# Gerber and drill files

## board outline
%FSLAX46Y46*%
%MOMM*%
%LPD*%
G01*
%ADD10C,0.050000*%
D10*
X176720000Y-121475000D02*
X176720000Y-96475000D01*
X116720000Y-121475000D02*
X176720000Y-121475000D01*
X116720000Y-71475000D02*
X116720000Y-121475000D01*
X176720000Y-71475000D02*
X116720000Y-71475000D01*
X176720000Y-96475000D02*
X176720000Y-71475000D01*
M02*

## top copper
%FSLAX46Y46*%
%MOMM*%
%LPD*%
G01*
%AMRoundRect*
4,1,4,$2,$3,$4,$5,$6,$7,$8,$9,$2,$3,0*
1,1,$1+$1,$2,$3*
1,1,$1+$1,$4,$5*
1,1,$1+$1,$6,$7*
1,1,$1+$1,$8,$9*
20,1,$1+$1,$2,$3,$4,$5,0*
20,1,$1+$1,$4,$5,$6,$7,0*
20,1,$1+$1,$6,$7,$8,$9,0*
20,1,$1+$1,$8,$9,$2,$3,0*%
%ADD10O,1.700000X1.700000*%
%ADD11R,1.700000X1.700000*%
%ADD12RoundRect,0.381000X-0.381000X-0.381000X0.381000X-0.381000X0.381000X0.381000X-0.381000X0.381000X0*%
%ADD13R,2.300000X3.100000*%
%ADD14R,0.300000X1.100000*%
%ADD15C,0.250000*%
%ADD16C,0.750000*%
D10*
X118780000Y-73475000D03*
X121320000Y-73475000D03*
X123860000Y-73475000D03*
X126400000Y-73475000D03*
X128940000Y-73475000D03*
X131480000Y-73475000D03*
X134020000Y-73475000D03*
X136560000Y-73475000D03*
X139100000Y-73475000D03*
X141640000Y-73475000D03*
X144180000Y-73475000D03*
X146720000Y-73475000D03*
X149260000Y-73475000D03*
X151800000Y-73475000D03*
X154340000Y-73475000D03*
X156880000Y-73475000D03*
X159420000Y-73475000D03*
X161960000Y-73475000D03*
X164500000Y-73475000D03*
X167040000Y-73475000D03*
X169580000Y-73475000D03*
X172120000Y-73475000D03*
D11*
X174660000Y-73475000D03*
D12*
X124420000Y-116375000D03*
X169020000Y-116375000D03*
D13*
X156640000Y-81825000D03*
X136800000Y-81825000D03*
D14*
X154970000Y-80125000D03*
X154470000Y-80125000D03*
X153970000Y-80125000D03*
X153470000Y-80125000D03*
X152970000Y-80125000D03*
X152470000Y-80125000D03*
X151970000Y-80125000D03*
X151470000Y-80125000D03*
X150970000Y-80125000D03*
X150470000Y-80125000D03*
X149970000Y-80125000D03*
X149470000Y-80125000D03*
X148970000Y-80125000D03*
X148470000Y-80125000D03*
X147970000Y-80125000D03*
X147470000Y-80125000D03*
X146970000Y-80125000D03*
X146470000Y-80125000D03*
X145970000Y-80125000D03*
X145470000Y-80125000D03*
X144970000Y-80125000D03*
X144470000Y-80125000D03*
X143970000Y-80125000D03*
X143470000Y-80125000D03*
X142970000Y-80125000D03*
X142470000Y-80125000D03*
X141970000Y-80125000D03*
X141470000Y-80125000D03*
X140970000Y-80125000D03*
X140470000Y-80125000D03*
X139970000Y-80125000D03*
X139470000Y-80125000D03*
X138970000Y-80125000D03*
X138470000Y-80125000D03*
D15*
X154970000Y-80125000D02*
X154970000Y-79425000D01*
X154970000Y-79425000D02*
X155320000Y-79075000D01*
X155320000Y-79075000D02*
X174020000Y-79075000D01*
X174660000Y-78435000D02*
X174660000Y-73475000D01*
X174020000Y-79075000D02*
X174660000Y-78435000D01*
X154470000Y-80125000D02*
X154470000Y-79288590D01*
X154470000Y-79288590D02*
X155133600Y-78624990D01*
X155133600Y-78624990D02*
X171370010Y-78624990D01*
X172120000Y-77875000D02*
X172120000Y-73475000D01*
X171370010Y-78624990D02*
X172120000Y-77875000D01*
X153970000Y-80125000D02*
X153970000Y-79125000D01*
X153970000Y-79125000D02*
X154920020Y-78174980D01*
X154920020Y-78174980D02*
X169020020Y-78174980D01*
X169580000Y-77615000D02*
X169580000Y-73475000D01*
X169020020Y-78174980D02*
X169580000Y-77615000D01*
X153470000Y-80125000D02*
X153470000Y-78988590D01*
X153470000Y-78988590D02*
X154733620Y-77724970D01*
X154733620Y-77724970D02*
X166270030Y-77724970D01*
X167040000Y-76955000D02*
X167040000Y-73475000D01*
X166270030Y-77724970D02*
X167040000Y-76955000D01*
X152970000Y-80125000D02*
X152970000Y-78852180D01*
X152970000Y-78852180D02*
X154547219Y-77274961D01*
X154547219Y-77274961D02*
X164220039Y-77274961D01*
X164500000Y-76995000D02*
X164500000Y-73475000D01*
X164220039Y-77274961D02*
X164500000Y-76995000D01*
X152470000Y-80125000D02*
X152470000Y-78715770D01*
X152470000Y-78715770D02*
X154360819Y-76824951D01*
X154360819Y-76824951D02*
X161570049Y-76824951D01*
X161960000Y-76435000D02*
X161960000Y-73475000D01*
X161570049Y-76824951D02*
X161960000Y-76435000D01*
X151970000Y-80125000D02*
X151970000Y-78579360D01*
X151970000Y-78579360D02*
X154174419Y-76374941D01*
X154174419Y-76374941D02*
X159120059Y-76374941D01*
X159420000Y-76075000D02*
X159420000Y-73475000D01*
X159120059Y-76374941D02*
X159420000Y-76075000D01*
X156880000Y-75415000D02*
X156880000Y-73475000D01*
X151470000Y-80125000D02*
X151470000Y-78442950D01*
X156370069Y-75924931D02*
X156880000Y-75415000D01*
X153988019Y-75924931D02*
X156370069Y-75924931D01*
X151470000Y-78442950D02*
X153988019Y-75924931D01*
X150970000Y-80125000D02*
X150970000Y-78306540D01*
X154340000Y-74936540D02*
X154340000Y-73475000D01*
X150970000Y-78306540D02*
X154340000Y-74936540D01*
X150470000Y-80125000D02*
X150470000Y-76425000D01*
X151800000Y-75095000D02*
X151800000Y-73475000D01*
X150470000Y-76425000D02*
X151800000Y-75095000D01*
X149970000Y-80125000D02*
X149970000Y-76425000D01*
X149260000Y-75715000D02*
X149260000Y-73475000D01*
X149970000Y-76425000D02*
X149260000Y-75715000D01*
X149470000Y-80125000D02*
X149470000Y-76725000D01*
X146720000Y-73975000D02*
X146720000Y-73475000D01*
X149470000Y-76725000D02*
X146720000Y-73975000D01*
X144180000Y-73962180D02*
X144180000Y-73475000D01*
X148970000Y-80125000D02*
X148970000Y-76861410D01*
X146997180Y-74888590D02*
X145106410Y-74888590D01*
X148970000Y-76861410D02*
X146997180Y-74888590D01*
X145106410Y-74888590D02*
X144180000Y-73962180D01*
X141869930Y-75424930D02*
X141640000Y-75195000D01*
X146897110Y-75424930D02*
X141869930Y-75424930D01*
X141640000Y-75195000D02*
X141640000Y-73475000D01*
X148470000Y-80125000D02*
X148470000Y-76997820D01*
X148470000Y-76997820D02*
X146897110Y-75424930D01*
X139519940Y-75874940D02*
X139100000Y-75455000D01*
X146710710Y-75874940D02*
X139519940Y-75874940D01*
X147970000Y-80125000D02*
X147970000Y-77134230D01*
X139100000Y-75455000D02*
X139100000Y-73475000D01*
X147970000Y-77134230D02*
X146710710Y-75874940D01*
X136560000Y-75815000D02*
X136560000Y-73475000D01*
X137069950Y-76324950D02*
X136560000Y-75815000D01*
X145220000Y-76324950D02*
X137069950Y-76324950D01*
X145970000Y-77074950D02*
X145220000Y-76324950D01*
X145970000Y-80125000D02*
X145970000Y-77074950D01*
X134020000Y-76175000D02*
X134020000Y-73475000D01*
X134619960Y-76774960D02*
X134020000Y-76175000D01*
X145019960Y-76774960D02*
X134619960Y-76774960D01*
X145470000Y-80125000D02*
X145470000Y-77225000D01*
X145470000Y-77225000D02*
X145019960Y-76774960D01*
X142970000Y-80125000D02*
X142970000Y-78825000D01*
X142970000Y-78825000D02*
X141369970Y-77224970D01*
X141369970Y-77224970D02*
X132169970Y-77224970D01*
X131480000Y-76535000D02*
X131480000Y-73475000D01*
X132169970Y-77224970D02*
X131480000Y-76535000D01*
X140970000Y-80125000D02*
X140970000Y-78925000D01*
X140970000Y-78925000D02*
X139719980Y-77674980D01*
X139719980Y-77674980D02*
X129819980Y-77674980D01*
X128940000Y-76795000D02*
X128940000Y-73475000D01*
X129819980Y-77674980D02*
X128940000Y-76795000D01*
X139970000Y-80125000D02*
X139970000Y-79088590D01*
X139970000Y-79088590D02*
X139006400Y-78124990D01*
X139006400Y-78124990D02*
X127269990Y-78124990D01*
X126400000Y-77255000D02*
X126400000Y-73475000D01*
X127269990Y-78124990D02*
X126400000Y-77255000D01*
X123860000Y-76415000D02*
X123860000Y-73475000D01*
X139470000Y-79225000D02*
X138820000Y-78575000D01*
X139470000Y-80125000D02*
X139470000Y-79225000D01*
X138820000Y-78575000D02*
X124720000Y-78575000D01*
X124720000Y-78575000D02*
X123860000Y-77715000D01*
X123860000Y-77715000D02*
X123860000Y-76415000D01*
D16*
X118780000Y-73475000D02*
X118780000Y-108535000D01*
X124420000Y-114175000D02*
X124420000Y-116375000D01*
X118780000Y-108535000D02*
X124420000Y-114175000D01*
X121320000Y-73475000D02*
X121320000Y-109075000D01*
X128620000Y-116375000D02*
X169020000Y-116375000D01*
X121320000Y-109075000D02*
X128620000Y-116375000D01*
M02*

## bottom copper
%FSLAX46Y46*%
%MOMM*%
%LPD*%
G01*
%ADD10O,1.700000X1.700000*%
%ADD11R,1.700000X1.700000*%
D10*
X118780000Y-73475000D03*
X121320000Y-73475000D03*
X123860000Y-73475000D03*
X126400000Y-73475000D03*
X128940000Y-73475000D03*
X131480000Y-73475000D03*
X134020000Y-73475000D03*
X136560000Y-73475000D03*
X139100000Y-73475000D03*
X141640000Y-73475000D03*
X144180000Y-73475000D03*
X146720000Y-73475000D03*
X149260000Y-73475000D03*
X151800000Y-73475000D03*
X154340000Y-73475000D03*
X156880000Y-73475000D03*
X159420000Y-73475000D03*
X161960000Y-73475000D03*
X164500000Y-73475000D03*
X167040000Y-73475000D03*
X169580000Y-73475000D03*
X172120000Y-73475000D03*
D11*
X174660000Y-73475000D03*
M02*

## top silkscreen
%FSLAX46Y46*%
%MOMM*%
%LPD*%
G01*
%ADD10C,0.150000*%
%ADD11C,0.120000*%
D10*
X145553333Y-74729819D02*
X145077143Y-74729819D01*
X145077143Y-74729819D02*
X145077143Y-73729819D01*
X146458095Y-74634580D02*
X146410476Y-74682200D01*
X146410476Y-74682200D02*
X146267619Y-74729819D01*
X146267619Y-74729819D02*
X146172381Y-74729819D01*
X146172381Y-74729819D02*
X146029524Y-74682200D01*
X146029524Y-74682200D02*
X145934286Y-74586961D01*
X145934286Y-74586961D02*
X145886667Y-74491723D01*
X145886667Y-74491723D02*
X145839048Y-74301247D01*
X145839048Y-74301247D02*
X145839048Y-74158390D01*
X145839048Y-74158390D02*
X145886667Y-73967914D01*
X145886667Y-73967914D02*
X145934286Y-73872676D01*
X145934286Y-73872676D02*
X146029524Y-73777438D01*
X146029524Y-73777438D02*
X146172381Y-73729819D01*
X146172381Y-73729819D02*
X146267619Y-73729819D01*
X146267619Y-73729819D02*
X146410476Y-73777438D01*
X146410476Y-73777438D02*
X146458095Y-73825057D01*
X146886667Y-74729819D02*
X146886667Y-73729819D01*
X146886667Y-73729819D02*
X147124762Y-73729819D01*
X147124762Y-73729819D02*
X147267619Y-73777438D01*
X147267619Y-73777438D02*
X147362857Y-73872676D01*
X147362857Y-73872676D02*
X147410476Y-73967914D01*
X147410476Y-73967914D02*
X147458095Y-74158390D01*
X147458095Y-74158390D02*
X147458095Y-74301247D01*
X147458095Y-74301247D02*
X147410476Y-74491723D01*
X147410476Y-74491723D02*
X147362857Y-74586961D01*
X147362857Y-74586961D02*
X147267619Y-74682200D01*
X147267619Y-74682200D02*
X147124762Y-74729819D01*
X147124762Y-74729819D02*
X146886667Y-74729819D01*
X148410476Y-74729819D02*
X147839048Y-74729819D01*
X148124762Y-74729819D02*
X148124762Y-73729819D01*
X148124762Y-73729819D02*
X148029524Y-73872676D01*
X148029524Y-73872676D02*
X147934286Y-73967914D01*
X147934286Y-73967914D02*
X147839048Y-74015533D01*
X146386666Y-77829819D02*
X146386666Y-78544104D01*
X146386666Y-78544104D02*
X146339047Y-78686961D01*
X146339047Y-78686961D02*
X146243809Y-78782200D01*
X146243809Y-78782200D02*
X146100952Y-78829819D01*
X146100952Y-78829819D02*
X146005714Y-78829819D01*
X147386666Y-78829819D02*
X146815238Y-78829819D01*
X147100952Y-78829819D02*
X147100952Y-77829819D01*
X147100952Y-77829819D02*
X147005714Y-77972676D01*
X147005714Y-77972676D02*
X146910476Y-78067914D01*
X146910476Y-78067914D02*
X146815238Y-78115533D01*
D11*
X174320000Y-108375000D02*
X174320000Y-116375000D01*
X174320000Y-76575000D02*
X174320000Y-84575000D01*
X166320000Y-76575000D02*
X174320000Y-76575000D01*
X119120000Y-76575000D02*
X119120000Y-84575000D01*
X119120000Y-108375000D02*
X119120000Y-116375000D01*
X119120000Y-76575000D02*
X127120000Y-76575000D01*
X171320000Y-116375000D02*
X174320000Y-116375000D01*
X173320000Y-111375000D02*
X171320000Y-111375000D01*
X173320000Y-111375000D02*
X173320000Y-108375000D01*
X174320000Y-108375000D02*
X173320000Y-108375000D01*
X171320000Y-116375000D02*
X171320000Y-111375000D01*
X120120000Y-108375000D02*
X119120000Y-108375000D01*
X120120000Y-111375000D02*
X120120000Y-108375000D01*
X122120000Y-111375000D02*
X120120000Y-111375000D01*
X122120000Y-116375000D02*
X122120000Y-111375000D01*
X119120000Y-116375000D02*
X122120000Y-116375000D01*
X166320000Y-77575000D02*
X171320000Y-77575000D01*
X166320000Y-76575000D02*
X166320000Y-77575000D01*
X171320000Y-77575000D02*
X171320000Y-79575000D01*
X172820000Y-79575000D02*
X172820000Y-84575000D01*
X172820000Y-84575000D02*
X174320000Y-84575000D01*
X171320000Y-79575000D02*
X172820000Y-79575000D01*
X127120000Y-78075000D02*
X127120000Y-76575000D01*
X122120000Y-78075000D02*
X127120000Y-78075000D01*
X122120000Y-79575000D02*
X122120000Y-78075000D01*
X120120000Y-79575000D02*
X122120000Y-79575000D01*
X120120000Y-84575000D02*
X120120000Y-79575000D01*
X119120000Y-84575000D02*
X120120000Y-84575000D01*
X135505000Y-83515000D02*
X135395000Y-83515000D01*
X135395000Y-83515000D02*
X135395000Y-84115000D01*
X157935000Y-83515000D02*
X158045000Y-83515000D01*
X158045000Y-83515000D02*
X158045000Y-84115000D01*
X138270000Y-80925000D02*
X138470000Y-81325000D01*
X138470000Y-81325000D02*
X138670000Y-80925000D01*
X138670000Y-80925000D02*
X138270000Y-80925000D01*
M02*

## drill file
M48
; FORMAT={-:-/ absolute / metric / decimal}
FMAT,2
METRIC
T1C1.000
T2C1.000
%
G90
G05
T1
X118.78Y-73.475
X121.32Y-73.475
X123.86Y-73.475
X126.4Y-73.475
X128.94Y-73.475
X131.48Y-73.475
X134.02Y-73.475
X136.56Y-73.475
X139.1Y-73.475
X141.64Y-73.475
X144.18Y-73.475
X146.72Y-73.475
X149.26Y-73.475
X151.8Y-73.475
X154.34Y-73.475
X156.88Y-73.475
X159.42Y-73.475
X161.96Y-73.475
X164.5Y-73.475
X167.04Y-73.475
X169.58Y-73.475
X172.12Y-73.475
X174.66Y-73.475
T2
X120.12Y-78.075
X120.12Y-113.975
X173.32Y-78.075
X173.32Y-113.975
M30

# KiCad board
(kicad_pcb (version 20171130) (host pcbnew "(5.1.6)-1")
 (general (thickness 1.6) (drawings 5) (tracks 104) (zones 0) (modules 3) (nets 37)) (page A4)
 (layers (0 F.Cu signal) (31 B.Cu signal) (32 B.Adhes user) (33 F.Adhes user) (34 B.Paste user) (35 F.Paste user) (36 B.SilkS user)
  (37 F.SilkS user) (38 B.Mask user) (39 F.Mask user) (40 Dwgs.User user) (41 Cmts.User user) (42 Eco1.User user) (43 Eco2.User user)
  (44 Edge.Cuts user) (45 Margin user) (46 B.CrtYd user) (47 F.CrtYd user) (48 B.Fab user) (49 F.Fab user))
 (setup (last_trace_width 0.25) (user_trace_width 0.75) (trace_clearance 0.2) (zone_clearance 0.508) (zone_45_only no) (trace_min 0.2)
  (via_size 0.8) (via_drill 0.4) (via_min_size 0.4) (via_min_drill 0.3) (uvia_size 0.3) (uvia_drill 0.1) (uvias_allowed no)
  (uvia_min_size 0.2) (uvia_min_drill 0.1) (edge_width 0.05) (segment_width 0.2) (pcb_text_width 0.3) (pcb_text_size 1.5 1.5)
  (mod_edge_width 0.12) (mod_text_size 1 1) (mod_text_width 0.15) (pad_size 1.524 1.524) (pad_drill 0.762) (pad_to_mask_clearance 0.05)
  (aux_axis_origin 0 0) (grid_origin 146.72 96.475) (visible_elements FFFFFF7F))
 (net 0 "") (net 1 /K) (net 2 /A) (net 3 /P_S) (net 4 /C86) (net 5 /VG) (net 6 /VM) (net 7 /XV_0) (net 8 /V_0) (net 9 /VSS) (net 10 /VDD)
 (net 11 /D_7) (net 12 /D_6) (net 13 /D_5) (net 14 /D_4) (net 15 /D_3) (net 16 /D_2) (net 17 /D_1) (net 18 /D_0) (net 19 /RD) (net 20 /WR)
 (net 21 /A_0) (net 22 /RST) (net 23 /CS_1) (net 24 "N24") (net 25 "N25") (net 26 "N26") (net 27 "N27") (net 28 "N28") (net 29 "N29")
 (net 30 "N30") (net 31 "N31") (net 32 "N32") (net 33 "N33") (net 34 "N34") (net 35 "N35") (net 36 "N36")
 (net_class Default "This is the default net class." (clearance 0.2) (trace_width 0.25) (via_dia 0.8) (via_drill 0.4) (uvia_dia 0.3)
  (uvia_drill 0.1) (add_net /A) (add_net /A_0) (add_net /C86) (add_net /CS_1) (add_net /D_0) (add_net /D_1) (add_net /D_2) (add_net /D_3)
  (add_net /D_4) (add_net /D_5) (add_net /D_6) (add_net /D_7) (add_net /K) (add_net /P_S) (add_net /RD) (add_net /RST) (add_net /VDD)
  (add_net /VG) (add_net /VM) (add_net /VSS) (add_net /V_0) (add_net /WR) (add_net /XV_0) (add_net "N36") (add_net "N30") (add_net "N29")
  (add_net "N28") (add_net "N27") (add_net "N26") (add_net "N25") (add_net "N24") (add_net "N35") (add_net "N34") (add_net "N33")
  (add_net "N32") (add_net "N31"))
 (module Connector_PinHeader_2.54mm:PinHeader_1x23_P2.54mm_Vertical (layer B.Cu) (at 174.66 73.475 90)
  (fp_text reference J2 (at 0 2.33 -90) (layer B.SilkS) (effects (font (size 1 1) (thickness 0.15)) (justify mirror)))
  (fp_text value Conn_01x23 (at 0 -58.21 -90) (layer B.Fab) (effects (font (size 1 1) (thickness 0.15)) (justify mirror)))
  (pad 23 thru_hole oval (at 0 -55.88 90) (size 1.7 1.7) (drill 1) (layers *.Cu *.Mask) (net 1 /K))
  (pad 22 thru_hole oval (at 0 -53.34 90) (size 1.7 1.7) (drill 1) (layers *.Cu *.Mask) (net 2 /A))
  (pad 21 thru_hole oval (at 0 -50.8 90) (size 1.7 1.7) (drill 1) (layers *.Cu *.Mask) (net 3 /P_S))
  (pad 20 thru_hole oval (at 0 -48.26 90) (size 1.7 1.7) (drill 1) (layers *.Cu *.Mask) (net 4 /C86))
  (pad 19 thru_hole oval (at 0 -45.72 90) (size 1.7 1.7) (drill 1) (layers *.Cu *.Mask) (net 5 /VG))
  (pad 18 thru_hole oval (at 0 -43.18 90) (size 1.7 1.7) (drill 1) (layers *.Cu *.Mask) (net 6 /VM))
  (pad 17 thru_hole oval (at 0 -40.64 90) (size 1.7 1.7) (drill 1) (layers *.Cu *.Mask) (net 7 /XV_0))
  (pad 16 thru_hole oval (at 0 -38.1 90) (size 1.7 1.7) (drill 1) (layers *.Cu *.Mask) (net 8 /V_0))
  (pad 15 thru_hole oval (at 0 -35.56 90) (size 1.7 1.7) (drill 1) (layers *.Cu *.Mask) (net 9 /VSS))
  (pad 14 thru_hole oval (at 0 -33.02 90) (size 1.7 1.7) (drill 1) (layers *.Cu *.Mask) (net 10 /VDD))
  (pad 13 thru_hole oval (at 0 -30.48 90) (size 1.7 1.7) (drill 1) (layers *.Cu *.Mask) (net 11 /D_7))
  (pad 12 thru_hole oval (at 0 -27.94 90) (size 1.7 1.7) (drill 1) (layers *.Cu *.Mask) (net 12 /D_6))
  (pad 11 thru_hole oval (at 0 -25.4 90) (size 1.7 1.7) (drill 1) (layers *.Cu *.Mask) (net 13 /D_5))
  (pad 10 thru_hole oval (at 0 -22.86 90) (size 1.7 1.7) (drill 1) (layers *.Cu *.Mask) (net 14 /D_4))
  (pad 9 thru_hole oval (at 0 -20.32 90) (size 1.7 1.7) (drill 1) (layers *.Cu *.Mask) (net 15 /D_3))
  (pad 8 thru_hole oval (at 0 -17.78 90) (size 1.7 1.7) (drill 1) (layers *.Cu *.Mask) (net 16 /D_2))
  (pad 7 thru_hole oval (at 0 -15.24 90) (size 1.7 1.7) (drill 1) (layers *.Cu *.Mask) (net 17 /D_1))
  (pad 6 thru_hole oval (at 0 -12.7 90) (size 1.7 1.7) (drill 1) (layers *.Cu *.Mask) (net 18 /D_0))
  (pad 5 thru_hole oval (at 0 -10.16 90) (size 1.7 1.7) (drill 1) (layers *.Cu *.Mask) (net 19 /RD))
  (pad 4 thru_hole oval (at 0 -7.62 90) (size 1.7 1.7) (drill 1) (layers *.Cu *.Mask) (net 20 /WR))
  (pad 3 thru_hole oval (at 0 -5.08 90) (size 1.7 1.7) (drill 1) (layers *.Cu *.Mask) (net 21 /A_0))
  (pad 2 thru_hole oval (at 0 -2.54 90) (size 1.7 1.7) (drill 1) (layers *.Cu *.Mask) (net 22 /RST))
  (pad 1 thru_hole rect (at 0 0 90) (size 1.7 1.7) (drill 1) (layers *.Cu *.Mask) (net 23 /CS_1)))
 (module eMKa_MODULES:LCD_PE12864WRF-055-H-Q (layer F.Cu) (at 146.72 96.475)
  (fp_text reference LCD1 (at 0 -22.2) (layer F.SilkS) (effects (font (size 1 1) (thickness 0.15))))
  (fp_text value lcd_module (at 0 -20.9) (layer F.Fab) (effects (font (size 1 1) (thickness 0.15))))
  (fp_line (start 27.6 11.9) (end 27.6 19.9) (layer F.SilkS) (width 0.12))
  (fp_line (start 27.6 -19.9) (end 27.6 -11.9) (layer F.SilkS) (width 0.12))
  (fp_line (start 19.6 -19.9) (end 27.6 -19.9) (layer F.SilkS) (width 0.12))
  (fp_line (start -27.6 -19.9) (end -27.6 -11.9) (layer F.SilkS) (width 0.12))
  (fp_line (start -27.6 11.9) (end -27.6 19.9) (layer F.SilkS) (width 0.12))
  (fp_line (start -27.6 -19.9) (end -19.6 -19.9) (layer F.SilkS) (width 0.12))
  (fp_line (start 24.6 19.9) (end 27.6 19.9) (layer F.SilkS) (width 0.12))
  (fp_line (start 26.6 14.9) (end 24.6 14.9) (layer F.SilkS) (width 0.12))
  (fp_line (start 26.6 14.9) (end 26.6 11.9) (layer F.SilkS) (width 0.12))
  (fp_line (start 27.6 11.9) (end 26.6 11.9) (layer F.SilkS) (width 0.12))
  (fp_line (start 24.6 19.9) (end 24.6 14.9) (layer F.SilkS) (width 0.12))
  (fp_line (start -26.6 11.9) (end -27.6 11.9) (layer F.SilkS) (width 0.12))
  (fp_line (start -26.6 14.9) (end -26.6 11.9) (layer F.SilkS) (width 0.12))
  (fp_line (start -24.6 14.9) (end -26.6 14.9) (layer F.SilkS) (width 0.12))
  (fp_line (start -24.6 19.9) (end -24.6 14.9) (layer F.SilkS) (width 0.12))
  (fp_line (start -27.6 19.9) (end -24.6 19.9) (layer F.SilkS) (width 0.12))
  (fp_line (start 19.6 -18.9) (end 24.6 -18.9) (layer F.SilkS) (width 0.12))
  (fp_line (start 19.6 -19.9) (end 19.6 -18.9) (layer F.SilkS) (width 0.12))
  (fp_line (start 24.6 -18.9) (end 24.6 -16.9) (layer F.SilkS) (width 0.12))
  (fp_line (start 26.1 -16.9) (end 26.1 -11.9) (layer F.SilkS) (width 0.12))
  (fp_line (start 26.1 -11.9) (end 27.6 -11.9) (layer F.SilkS) (width 0.12))
  (fp_line (start 24.6 -16.9) (end 26.1 -16.9) (layer F.SilkS) (width 0.12))
  (fp_line (start -19.6 -18.4) (end -19.6 -19.9) (layer F.SilkS) (width 0.12))
  (fp_line (start -24.6 -18.4) (end -19.6 -18.4) (layer F.SilkS) (width 0.12))
  (fp_line (start -24.6 -16.9) (end -24.6 -18.4) (layer F.SilkS) (width 0.12))
  (fp_line (start -26.6 -16.9) (end -24.6 -16.9) (layer F.SilkS) (width 0.12))
  (fp_line (start -26.6 -11.9) (end -26.6 -16.9) (layer F.SilkS) (width 0.12))
  (fp_line (start -27.6 -11.9) (end -26.6 -11.9) (layer F.SilkS) (width 0.12))
  (pad 1 smd roundrect (at -22.3 19.9) (size 1.524 1.524) (layers F.Cu F.Paste F.Mask) (roundrect_rratio 0.25) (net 1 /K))
  (pad 2 smd roundrect (at 22.3 19.9) (size 1.524 1.524) (layers F.Cu F.Paste F.Mask) (roundrect_rratio 0.25) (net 2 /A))
  (pad "" np_thru_hole circle (at -26.6 17.5) (size 1 1) (drill 1) (layers *.Cu *.Mask))
  (pad "" np_thru_hole circle (at 26.6 17.5) (size 1 1) (drill 1) (layers *.Cu *.Mask))
  (pad "" np_thru_hole circle (at 26.6 -18.4) (size 1 1) (drill 1) (layers *.Cu *.Mask))
  (pad "" np_thru_hole circle (at -26.6 -18.4) (size 1 1) (drill 1) (layers *.Cu *.Mask)))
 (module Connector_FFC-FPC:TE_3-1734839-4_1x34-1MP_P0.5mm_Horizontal (layer F.Cu) (at 146.72 81.475)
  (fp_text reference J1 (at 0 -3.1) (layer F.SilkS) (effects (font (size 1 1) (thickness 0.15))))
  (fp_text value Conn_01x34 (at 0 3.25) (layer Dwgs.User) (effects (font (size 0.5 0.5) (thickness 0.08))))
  (fp_line (start -11.215 2.04) (end -11.325 2.04) (layer F.SilkS) (width 0.12))
  (fp_line (start -11.325 2.04) (end -11.325 2.64) (layer F.SilkS) (width 0.12))
  (fp_line (start 11.215 2.04) (end 11.325 2.04) (layer F.SilkS) (width 0.12))
  (fp_line (start 11.325 2.04) (end 11.325 2.64) (layer F.SilkS) (width 0.12))
  (fp_line (start -8.45 -0.55) (end -8.25 -0.15) (layer F.SilkS) (width 0.12))
  (fp_line (start -8.25 -0.15) (end -8.05 -0.55) (layer F.SilkS) (width 0.12))
  (fp_line (start -8.05 -0.55) (end -8.45 -0.55) (layer F.SilkS) (width 0.12))
  (pad MP smd rect (at 9.92 0.35) (size 2.3 3.1) (layers F.Cu F.Paste F.Mask))
  (pad MP smd rect (at -9.92 0.35) (size 2.3 3.1) (layers F.Cu F.Paste F.Mask))
  (pad 34 smd rect (at 8.25 -1.35) (size 0.3 1.1) (layers F.Cu F.Paste F.Mask) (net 23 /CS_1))
  (pad 33 smd rect (at 7.75 -1.35) (size 0.3 1.1) (layers F.Cu F.Paste F.Mask) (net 22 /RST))
  (pad 32 smd rect (at 7.25 -1.35) (size 0.3 1.1) (layers F.Cu F.Paste F.Mask) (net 21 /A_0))
  (pad 31 smd rect (at 6.75 -1.35) (size 0.3 1.1) (layers F.Cu F.Paste F.Mask) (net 20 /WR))
  (pad 30 smd rect (at 6.25 -1.35) (size 0.3 1.1) (layers F.Cu F.Paste F.Mask) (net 19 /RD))
  (pad 29 smd rect (at 5.75 -1.35) (size 0.3 1.1) (layers F.Cu F.Paste F.Mask) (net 18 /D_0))
  (pad 28 smd rect (at 5.25 -1.35) (size 0.3 1.1) (layers F.Cu F.Paste F.Mask) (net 17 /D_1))
  (pad 27 smd rect (at 4.75 -1.35) (size 0.3 1.1) (layers F.Cu F.Paste F.Mask) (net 16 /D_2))
  (pad 26 smd rect (at 4.25 -1.35) (size 0.3 1.1) (layers F.Cu F.Paste F.Mask) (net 15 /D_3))
  (pad 25 smd rect (at 3.75 -1.35) (size 0.3 1.1) (layers F.Cu F.Paste F.Mask) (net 14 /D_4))
  (pad 24 smd rect (at 3.25 -1.35) (size 0.3 1.1) (layers F.Cu F.Paste F.Mask) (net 13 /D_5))
  (pad 23 smd rect (at 2.75 -1.35) (size 0.3 1.1) (layers F.Cu F.Paste F.Mask) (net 12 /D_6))
  (pad 22 smd rect (at 2.25 -1.35) (size 0.3 1.1) (layers F.Cu F.Paste F.Mask) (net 11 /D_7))
  (pad 21 smd rect (at 1.75 -1.35) (size 0.3 1.1) (layers F.Cu F.Paste F.Mask) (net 10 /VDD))
  (pad 20 smd rect (at 1.25 -1.35) (size 0.3 1.1) (layers F.Cu F.Paste F.Mask) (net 9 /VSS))
  (pad 19 smd rect (at 0.75 -1.35) (size 0.3 1.1) (layers F.Cu F.Paste F.Mask) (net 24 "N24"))
  (pad 18 smd rect (at 0.25 -1.35) (size 0.3 1.1) (layers F.Cu F.Paste F.Mask) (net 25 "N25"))
  (pad 17 smd rect (at -0.25 -1.35) (size 0.3 1.1) (layers F.Cu F.Paste F.Mask) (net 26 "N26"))
  (pad 16 smd rect (at -0.75 -1.35) (size 0.3 1.1) (layers F.Cu F.Paste F.Mask) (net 8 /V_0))
  (pad 15 smd rect (at -1.25 -1.35) (size 0.3 1.1) (layers F.Cu F.Paste F.Mask) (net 7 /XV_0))
  (pad 14 smd rect (at -1.75 -1.35) (size 0.3 1.1) (layers F.Cu F.Paste F.Mask) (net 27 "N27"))
  (pad 13 smd rect (at -2.25 -1.35) (size 0.3 1.1) (layers F.Cu F.Paste F.Mask) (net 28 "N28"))
  (pad 12 smd rect (at -2.75 -1.35) (size 0.3 1.1) (layers F.Cu F.Paste F.Mask) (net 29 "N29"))
  (pad 11 smd rect (at -3.25 -1.35) (size 0.3 1.1) (layers F.Cu F.Paste F.Mask) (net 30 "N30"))
  (pad 10 smd rect (at -3.75 -1.35) (size 0.3 1.1) (layers F.Cu F.Paste F.Mask) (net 6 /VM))
  (pad 9 smd rect (at -4.25 -1.35) (size 0.3 1.1) (layers F.Cu F.Paste F.Mask) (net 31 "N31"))
  (pad 8 smd rect (at -4.75 -1.35) (size 0.3 1.1) (layers F.Cu F.Paste F.Mask) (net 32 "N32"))
  (pad 7 smd rect (at -5.25 -1.35) (size 0.3 1.1) (layers F.Cu F.Paste F.Mask) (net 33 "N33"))
  (pad 6 smd rect (at -5.75 -1.35) (size 0.3 1.1) (layers F.Cu F.Paste F.Mask) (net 5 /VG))
  (pad 5 smd rect (at -6.25 -1.35) (size 0.3 1.1) (layers F.Cu F.Paste F.Mask) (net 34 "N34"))
  (pad 4 smd rect (at -6.75 -1.35) (size 0.3 1.1) (layers F.Cu F.Paste F.Mask) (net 4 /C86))
  (pad 3 smd rect (at -7.25 -1.35) (size 0.3 1.1) (layers F.Cu F.Paste F.Mask) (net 3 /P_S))
  (pad 2 smd rect (at -7.75 -1.35) (size 0.3 1.1) (layers F.Cu F.Paste F.Mask) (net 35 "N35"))
  (pad 1 smd rect (at -8.25 -1.35) (size 0.3 1.1) (layers F.Cu F.Paste F.Mask) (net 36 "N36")))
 (gr_line (start 176.72 121.475) (end 176.72 96.475) (layer Edge.Cuts) (width 0.05))
 (gr_line (start 116.72 121.475) (end 176.72 121.475) (layer Edge.Cuts) (width 0.05))
 (gr_line (start 116.72 71.475) (end 116.72 121.475) (layer Edge.Cuts) (width 0.05))
 (gr_line (start 176.72 71.475) (end 116.72 71.475) (layer Edge.Cuts) (width 0.05))
 (gr_line (start 176.72 96.475) (end 176.72 71.475) (layer Edge.Cuts) (width 0.05))
 (segment (start 154.97 80.125) (end 154.97 79.425) (width 0.25) (layer F.Cu) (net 23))
 (segment (start 154.97 79.425) (end 155.32 79.075) (width 0.25) (layer F.Cu) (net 23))
 (segment (start 155.32 79.075) (end 174.02 79.075) (width 0.25) (layer F.Cu) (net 23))
 (segment (start 174.66 78.435) (end 174.66 73.475) (width 0.25) (layer F.Cu) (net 23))
 (segment (start 174.02 79.075) (end 174.66 78.435) (width 0.25) (layer F.Cu) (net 23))
 (segment (start 154.47 80.125) (end 154.47 79.28859) (width 0.25) (layer F.Cu) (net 22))
 (segment (start 154.47 79.28859) (end 155.1336 78.62499) (width 0.25) (layer F.Cu) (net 22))
 (segment (start 155.1336 78.62499) (end 171.37001 78.62499) (width 0.25) (layer F.Cu) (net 22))
 (segment (start 172.12 77.875) (end 172.12 73.475) (width 0.25) (layer F.Cu) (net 22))
 (segment (start 171.37001 78.62499) (end 172.12 77.875) (width 0.25) (layer F.Cu) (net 22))
 (segment (start 153.97 80.125) (end 153.97 79.125) (width 0.25) (layer F.Cu) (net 21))
 (segment (start 153.97 79.125) (end 154.92002 78.17498) (width 0.25) (layer F.Cu) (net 21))
 (segment (start 154.92002 78.17498) (end 169.02002 78.17498) (width 0.25) (layer F.Cu) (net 21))
 (segment (start 169.58 77.615) (end 169.58 73.475) (width 0.25) (layer F.Cu) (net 21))
 (segment (start 169.02002 78.17498) (end 169.58 77.615) (width 0.25) (layer F.Cu) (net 21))
 (segment (start 153.47 80.125) (end 153.47 78.98859) (width 0.25) (layer F.Cu) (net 20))
 (segment (start 153.47 78.98859) (end 154.73362 77.72497) (width 0.25) (layer F.Cu) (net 20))
 (segment (start 154.73362 77.72497) (end 166.27003 77.72497) (width 0.25) (layer F.Cu) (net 20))
 (segment (start 167.04 76.955) (end 167.04 73.475) (width 0.25) (layer F.Cu) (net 20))
 (segment (start 166.27003 77.72497) (end 167.04 76.955) (width 0.25) (layer F.Cu) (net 20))
 (segment (start 152.97 80.125) (end 152.97 78.85218) (width 0.25) (layer F.Cu) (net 19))
 (segment (start 152.97 78.85218) (end 154.547219 77.274961) (width 0.25) (layer F.Cu) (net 19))
 (segment (start 154.547219 77.274961) (end 164.220039 77.274961) (width 0.25) (layer F.Cu) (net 19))
 (segment (start 164.5 76.995) (end 164.5 73.475) (width 0.25) (layer F.Cu) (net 19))
 (segment (start 164.220039 77.274961) (end 164.5 76.995) (width 0.25) (layer F.Cu) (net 19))
 (segment (start 152.47 80.125) (end 152.47 78.71577) (width 0.25) (layer F.Cu) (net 18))
 (segment (start 152.47 78.71577) (end 154.360819 76.824951) (width 0.25) (layer F.Cu) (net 18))
 (segment (start 154.360819 76.824951) (end 161.570049 76.824951) (width 0.25) (layer F.Cu) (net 18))
 (segment (start 161.96 76.435) (end 161.96 73.475) (width 0.25) (layer F.Cu) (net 18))
 (segment (start 161.570049 76.824951) (end 161.96 76.435) (width 0.25) (layer F.Cu) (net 18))
 (segment (start 151.97 80.125) (end 151.97 78.57936) (width 0.25) (layer F.Cu) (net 17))
 (segment (start 151.97 78.57936) (end 154.174419 76.374941) (width 0.25) (layer F.Cu) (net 17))
 (segment (start 154.174419 76.374941) (end 159.120059 76.374941) (width 0.25) (layer F.Cu) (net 17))
 (segment (start 159.42 76.075) (end 159.42 73.475) (width 0.25) (layer F.Cu) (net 17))
 (segment (start 159.120059 76.374941) (end 159.42 76.075) (width 0.25) (layer F.Cu) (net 17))
 (segment (start 156.88 75.415) (end 156.88 73.475) (width 0.25) (layer F.Cu) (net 16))
 (segment (start 151.47 80.125) (end 151.47 78.44295) (width 0.25) (layer F.Cu) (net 16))
 (segment (start 156.370069 75.924931) (end 156.88 75.415) (width 0.25) (layer F.Cu) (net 16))
 (segment (start 153.988019 75.924931) (end 156.370069 75.924931) (width 0.25) (layer F.Cu) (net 16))
 (segment (start 151.47 78.44295) (end 153.988019 75.924931) (width 0.25) (layer F.Cu) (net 16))
 (segment (start 150.97 80.125) (end 150.97 78.30654) (width 0.25) (layer F.Cu) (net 15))
 (segment (start 154.34 74.93654) (end 154.34 73.475) (width 0.25) (layer F.Cu) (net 15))
 (segment (start 150.97 78.30654) (end 154.34 74.93654) (width 0.25) (layer F.Cu) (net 15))
 (segment (start 150.47 80.125) (end 150.47 76.425) (width 0.25) (layer F.Cu) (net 14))
 (segment (start 151.8 75.095) (end 151.8 73.475) (width 0.25) (layer F.Cu) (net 14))
 (segment (start 150.47 76.425) (end 151.8 75.095) (width 0.25) (layer F.Cu) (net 14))
 (segment (start 149.97 80.125) (end 149.97 76.425) (width 0.25) (layer F.Cu) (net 13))
 (segment (start 149.26 75.715) (end 149.26 73.475) (width 0.25) (layer F.Cu) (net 13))
 (segment (start 149.97 76.425) (end 149.26 75.715) (width 0.25) (layer F.Cu) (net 13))
 (segment (start 149.47 80.125) (end 149.47 76.725) (width 0.25) (layer F.Cu) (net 12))
 (segment (start 146.72 73.975) (end 146.72 73.475) (width 0.25) (layer F.Cu) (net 12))
 (segment (start 149.47 76.725) (end 146.72 73.975) (width 0.25) (layer F.Cu) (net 12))
 (segment (start 144.18 73.96218) (end 144.18 73.475) (width 0.25) (layer F.Cu) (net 11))
 (segment (start 148.97 80.125) (end 148.97 76.86141) (width 0.25) (layer F.Cu) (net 11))
 (segment (start 146.99718 74.88859) (end 145.10641 74.88859) (width 0.25) (layer F.Cu) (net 11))
 (segment (start 148.97 76.86141) (end 146.99718 74.88859) (width 0.25) (layer F.Cu) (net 11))
 (segment (start 145.10641 74.88859) (end 144.18 73.96218) (width 0.25) (layer F.Cu) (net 11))
 (segment (start 141.86993 75.42493) (end 141.64 75.195) (width 0.25) (layer F.Cu) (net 10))
 (segment (start 146.89711 75.42493) (end 141.86993 75.42493) (width 0.25) (layer F.Cu) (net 10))
 (segment (start 141.64 75.195) (end 141.64 73.475) (width 0.25) (layer F.Cu) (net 10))
 (segment (start 148.47 80.125) (end 148.47 76.99782) (width 0.25) (layer F.Cu) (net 10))
 (segment (start 148.47 76.99782) (end 146.89711 75.42493) (width 0.25) (layer F.Cu) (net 10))
 (segment (start 139.51994 75.87494) (end 139.1 75.455) (width 0.25) (layer F.Cu) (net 9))
 (segment (start 146.71071 75.87494) (end 139.51994 75.87494) (width 0.25) (layer F.Cu) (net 9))
 (segment (start 147.97 80.125) (end 147.97 77.13423) (width 0.25) (layer F.Cu) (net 9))
 (segment (start 139.1 75.455) (end 139.1 73.475) (width 0.25) (layer F.Cu) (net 9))
 (segment (start 147.97 77.13423) (end 146.71071 75.87494) (width 0.25) (layer F.Cu) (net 9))
 (segment (start 136.56 75.815) (end 136.56 73.475) (width 0.25) (layer F.Cu) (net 8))
 (segment (start 137.06995 76.32495) (end 136.56 75.815) (width 0.25) (layer F.Cu) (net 8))
 (segment (start 145.22 76.32495) (end 137.06995 76.32495) (width 0.25) (layer F.Cu) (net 8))
 (segment (start 145.97 77.07495) (end 145.22 76.32495) (width 0.25) (layer F.Cu) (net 8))
 (segment (start 145.97 80.125) (end 145.97 77.07495) (width 0.25) (layer F.Cu) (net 8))
 (segment (start 134.02 76.175) (end 134.02 73.475) (width 0.25) (layer F.Cu) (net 7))
 (segment (start 134.61996 76.77496) (end 134.02 76.175) (width 0.25) (layer F.Cu) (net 7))
 (segment (start 145.01996 76.77496) (end 134.61996 76.77496) (width 0.25) (layer F.Cu) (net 7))
 (segment (start 145.47 80.125) (end 145.47 77.225) (width 0.25) (layer F.Cu) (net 7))
 (segment (start 145.47 77.225) (end 145.01996 76.77496) (width 0.25) (layer F.Cu) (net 7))
 (segment (start 142.97 80.125) (end 142.97 78.825) (width 0.25) (layer F.Cu) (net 6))
 (segment (start 142.97 78.825) (end 141.36997 77.22497) (width 0.25) (layer F.Cu) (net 6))
 (segment (start 141.36997 77.22497) (end 132.16997 77.22497) (width 0.25) (layer F.Cu) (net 6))
 (segment (start 131.48 76.535) (end 131.48 73.475) (width 0.25) (layer F.Cu) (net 6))
 (segment (start 132.16997 77.22497) (end 131.48 76.535) (width 0.25) (layer F.Cu) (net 6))
 (segment (start 140.97 80.125) (end 140.97 78.925) (width 0.25) (layer F.Cu) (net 5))
 (segment (start 140.97 78.925) (end 139.71998 77.67498) (width 0.25) (layer F.Cu) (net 5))
 (segment (start 139.71998 77.67498) (end 129.81998 77.67498) (width 0.25) (layer F.Cu) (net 5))
 (segment (start 128.94 76.795) (end 128.94 73.475) (width 0.25) (layer F.Cu) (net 5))
 (segment (start 129.81998 77.67498) (end 128.94 76.795) (width 0.25) (layer F.Cu) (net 5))
 (segment (start 139.97 80.125) (end 139.97 79.08859) (width 0.25) (layer F.Cu) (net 4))
 (segment (start 139.97 79.08859) (end 139.0064 78.12499) (width 0.25) (layer F.Cu) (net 4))
 (segment (start 139.0064 78.12499) (end 127.26999 78.12499) (width 0.25) (layer F.Cu) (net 4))
 (segment (start 126.4 77.255) (end 126.4 73.475) (width 0.25) (layer F.Cu) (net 4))
 (segment (start 127.26999 78.12499) (end 126.4 77.255) (width 0.25) (layer F.Cu) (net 4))
 (segment (start 123.86 76.415) (end 123.86 73.475) (width 0.25) (layer F.Cu) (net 3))
 (segment (start 139.47 79.225) (end 138.82 78.575) (width 0.25) (layer F.Cu) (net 3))
 (segment (start 139.47 80.125) (end 139.47 79.225) (width 0.25) (layer F.Cu) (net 3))
 (segment (start 138.82 78.575) (end 124.72 78.575) (width 0.25) (layer F.Cu) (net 3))
 (segment (start 124.72 78.575) (end 123.86 77.715) (width 0.25) (layer F.Cu) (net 3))
 (segment (start 123.86 77.715) (end 123.86 76.415) (width 0.25) (layer F.Cu) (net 3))
 (segment (start 118.78 73.475) (end 118.78 108.535) (width 0.75) (layer F.Cu) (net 1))
 (segment (start 124.42 114.175) (end 124.42 116.375) (width 0.75) (layer F.Cu) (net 1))
 (segment (start 118.78 108.535) (end 124.42 114.175) (width 0.75) (layer F.Cu) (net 1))
 (segment (start 121.32 73.475) (end 121.32 109.075) (width 0.75) (layer F.Cu) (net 2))
 (segment (start 128.62 116.375) (end 169.02 116.375) (width 0.75) (layer F.Cu) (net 2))
 (segment (start 121.32 109.075) (end 128.62 116.375) (width 0.75) (layer F.Cu) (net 2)))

